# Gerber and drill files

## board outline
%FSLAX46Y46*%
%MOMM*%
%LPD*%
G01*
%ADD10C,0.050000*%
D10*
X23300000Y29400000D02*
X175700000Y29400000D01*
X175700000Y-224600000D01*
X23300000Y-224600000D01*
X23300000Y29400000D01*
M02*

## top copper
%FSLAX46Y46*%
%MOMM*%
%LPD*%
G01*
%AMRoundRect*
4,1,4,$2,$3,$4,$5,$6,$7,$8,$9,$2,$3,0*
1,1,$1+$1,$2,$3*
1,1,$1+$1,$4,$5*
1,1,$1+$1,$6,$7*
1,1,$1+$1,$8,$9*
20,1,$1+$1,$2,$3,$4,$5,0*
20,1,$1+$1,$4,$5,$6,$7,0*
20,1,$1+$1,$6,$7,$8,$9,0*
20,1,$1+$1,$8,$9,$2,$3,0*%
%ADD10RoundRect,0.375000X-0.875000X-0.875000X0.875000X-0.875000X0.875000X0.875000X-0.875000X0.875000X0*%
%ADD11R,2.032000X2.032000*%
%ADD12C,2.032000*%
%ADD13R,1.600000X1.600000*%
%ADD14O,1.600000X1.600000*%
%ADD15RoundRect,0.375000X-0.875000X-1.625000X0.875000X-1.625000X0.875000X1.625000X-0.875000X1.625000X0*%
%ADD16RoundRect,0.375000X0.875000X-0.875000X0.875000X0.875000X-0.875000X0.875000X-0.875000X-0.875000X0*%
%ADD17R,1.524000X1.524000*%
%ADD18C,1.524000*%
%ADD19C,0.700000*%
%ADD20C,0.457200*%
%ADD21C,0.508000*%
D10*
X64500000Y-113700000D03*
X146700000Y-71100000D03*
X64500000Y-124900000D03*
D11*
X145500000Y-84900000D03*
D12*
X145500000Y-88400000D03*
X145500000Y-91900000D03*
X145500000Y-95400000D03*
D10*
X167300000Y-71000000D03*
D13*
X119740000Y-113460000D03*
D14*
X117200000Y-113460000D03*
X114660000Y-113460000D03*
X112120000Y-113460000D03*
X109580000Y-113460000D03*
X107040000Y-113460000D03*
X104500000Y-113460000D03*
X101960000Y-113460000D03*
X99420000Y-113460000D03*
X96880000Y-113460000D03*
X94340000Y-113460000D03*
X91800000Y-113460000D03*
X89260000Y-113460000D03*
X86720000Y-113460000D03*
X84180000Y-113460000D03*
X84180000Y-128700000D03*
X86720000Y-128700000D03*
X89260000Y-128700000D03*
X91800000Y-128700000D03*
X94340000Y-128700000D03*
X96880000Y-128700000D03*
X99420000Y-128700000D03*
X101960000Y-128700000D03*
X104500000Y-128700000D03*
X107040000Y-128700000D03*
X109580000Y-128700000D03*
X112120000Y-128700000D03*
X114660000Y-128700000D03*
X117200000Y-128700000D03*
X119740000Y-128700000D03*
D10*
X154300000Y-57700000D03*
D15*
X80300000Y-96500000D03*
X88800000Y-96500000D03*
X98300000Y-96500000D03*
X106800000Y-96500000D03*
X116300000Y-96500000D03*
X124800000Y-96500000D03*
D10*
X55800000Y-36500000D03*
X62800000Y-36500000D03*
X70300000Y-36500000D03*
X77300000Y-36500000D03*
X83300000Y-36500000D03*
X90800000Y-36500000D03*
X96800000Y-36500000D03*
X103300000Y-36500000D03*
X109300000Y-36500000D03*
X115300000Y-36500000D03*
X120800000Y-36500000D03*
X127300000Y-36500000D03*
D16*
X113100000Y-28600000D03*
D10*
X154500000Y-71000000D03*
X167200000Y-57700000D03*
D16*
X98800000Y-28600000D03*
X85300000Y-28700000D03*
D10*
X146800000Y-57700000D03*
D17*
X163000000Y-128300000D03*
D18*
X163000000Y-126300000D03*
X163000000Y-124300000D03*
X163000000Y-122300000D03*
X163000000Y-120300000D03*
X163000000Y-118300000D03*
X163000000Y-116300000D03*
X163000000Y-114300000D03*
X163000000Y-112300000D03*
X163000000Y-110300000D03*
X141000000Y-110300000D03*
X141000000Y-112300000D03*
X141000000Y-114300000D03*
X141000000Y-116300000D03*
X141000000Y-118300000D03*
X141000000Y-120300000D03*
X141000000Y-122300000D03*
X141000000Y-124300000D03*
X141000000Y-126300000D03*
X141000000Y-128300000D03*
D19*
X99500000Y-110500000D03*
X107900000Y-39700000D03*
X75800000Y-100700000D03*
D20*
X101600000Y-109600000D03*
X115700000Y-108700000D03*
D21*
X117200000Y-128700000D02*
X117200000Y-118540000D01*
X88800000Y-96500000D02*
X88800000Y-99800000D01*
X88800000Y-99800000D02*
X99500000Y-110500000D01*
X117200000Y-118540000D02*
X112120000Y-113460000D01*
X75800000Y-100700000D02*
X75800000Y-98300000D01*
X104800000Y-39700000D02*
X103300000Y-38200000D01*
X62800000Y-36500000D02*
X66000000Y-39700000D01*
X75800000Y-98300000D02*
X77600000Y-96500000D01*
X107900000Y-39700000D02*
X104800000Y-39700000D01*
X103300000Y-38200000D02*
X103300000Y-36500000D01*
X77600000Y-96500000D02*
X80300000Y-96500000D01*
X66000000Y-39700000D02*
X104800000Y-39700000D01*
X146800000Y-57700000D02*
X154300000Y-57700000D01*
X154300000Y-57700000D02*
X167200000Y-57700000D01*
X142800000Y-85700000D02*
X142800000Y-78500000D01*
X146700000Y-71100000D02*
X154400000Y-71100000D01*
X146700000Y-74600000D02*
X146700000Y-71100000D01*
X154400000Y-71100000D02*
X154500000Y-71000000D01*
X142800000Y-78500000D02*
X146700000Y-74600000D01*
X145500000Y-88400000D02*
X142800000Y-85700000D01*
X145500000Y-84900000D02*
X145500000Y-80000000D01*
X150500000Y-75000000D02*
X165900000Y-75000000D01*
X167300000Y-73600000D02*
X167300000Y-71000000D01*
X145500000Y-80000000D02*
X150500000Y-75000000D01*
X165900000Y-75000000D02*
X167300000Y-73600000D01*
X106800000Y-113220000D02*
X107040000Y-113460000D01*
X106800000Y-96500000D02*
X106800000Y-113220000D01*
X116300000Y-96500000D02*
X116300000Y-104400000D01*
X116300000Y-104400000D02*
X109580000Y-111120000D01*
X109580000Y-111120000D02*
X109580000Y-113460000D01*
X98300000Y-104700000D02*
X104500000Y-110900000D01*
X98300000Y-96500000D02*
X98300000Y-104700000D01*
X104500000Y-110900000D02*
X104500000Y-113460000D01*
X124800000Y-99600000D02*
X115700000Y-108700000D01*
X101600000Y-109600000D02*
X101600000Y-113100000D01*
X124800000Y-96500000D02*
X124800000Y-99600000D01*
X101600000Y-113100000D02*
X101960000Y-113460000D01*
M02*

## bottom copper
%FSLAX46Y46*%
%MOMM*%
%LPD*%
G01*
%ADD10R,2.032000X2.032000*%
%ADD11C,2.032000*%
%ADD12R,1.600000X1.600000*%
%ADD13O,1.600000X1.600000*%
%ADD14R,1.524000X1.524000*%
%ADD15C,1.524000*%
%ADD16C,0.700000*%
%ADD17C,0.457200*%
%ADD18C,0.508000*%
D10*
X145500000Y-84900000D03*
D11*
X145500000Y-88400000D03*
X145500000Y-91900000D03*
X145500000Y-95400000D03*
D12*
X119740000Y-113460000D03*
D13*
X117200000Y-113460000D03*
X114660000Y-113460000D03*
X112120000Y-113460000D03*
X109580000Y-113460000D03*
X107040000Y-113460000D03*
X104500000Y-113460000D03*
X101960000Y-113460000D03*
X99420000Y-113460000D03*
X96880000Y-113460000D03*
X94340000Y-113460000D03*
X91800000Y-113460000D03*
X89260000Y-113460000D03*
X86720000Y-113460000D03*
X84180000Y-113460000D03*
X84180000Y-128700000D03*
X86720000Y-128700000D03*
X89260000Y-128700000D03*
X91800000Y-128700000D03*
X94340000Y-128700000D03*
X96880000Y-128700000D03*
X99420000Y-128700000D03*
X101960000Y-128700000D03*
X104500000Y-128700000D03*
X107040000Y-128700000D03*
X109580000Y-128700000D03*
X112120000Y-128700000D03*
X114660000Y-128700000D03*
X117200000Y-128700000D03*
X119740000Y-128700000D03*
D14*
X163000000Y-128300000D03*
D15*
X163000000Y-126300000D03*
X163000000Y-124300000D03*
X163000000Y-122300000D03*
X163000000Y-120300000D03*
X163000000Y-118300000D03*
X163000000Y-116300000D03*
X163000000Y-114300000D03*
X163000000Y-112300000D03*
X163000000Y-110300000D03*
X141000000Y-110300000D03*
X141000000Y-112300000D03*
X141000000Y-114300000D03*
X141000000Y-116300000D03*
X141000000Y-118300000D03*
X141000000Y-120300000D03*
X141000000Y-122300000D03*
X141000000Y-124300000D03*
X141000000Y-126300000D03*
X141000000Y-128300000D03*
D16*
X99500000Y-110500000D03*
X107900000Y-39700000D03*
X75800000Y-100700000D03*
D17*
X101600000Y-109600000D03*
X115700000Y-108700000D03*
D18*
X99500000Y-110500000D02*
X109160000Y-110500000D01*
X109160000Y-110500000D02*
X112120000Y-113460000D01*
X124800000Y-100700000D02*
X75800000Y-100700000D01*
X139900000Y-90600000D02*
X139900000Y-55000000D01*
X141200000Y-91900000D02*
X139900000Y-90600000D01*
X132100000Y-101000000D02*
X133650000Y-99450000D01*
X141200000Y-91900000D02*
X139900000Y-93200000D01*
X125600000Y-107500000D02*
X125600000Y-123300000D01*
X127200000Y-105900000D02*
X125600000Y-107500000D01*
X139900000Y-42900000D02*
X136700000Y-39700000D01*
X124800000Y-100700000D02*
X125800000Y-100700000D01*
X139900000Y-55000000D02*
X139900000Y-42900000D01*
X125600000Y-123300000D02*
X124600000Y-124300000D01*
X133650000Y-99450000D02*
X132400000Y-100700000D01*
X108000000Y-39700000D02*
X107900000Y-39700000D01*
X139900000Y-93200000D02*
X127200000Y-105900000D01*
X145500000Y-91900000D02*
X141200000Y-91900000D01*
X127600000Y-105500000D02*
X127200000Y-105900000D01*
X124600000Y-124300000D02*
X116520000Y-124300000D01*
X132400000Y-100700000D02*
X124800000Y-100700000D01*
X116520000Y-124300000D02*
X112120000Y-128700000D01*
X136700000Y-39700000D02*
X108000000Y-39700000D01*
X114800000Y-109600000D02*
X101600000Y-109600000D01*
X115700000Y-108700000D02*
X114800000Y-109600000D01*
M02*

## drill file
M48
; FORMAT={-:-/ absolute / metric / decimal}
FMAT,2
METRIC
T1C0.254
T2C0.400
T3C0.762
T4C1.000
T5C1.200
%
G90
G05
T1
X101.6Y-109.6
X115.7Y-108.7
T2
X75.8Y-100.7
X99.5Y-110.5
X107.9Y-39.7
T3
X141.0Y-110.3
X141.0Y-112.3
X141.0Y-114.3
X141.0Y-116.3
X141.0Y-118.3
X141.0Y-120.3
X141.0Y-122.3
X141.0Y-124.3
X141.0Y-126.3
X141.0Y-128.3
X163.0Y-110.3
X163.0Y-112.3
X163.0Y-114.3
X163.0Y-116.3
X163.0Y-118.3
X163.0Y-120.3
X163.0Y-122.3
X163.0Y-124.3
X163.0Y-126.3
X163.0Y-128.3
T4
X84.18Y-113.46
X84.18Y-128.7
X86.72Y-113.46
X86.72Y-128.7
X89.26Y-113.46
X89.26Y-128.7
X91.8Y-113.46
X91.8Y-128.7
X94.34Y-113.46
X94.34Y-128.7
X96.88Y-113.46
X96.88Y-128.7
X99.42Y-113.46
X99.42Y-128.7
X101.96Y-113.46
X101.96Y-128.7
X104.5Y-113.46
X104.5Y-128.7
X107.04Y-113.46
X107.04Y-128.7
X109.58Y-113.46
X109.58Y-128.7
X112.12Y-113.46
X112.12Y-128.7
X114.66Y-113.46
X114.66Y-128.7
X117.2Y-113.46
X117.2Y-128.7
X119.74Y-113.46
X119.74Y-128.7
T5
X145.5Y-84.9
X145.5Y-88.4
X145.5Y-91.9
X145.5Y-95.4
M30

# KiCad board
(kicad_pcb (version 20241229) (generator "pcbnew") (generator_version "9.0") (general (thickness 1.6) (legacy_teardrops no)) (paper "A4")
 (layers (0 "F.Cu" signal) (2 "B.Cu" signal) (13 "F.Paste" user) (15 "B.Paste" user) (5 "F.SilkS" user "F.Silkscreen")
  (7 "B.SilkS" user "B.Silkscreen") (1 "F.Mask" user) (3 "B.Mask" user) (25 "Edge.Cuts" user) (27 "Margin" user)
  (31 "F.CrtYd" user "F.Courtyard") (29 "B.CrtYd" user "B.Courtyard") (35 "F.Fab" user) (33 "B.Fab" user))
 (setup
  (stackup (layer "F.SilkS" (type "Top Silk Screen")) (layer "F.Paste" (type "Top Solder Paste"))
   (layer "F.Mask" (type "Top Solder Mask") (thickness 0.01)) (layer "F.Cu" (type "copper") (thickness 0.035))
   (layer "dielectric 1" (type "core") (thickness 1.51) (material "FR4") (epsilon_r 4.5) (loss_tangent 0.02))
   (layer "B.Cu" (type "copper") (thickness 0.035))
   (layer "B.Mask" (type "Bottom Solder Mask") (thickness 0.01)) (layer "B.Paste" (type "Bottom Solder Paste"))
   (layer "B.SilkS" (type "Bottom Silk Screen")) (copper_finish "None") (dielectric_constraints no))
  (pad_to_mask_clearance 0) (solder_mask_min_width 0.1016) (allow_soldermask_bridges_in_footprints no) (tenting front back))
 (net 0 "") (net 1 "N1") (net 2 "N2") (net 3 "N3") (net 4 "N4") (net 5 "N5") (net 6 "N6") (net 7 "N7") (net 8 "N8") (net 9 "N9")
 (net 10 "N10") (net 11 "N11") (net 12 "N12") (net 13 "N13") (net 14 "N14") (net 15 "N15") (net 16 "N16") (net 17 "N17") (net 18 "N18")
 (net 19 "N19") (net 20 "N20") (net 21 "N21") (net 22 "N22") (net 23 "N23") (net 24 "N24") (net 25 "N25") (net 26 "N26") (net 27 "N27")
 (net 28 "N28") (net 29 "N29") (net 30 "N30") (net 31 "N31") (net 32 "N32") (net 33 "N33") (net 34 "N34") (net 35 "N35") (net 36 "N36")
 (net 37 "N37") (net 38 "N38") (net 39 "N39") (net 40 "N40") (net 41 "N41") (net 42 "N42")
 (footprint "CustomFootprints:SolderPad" (layer "F.Cu") (at 64.5 113.7)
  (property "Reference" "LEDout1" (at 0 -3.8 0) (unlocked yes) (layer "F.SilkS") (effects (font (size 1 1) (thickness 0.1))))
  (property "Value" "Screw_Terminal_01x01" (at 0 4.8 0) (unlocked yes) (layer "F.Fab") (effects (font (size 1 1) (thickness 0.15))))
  (pad "1" smd roundrect (at 0 0) (size 2.5 2.5) (layers "F.Cu" "F.Mask" "F.Paste") (roundrect_rratio 0.15) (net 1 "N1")))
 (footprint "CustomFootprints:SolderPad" (layer "F.Cu") (at 146.7 71.1)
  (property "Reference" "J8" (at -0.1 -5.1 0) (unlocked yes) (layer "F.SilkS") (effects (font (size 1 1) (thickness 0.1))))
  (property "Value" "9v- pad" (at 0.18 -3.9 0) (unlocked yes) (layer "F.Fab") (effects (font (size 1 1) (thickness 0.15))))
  (pad "1" smd roundrect (at 0 0) (size 2.5 2.5) (layers "F.Cu" "F.Mask" "F.Paste") (roundrect_rratio 0.15) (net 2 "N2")))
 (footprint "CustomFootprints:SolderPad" (layer "F.Cu") (at 64.5 124.9)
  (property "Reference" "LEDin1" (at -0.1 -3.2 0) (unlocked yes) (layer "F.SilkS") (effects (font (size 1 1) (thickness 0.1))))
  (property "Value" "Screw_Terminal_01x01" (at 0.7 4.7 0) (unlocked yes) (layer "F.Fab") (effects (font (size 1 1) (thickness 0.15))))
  (pad "1" smd roundrect (at 0 0) (size 2.5 2.5) (layers "F.Cu" "F.Mask" "F.Paste") (roundrect_rratio 0.15) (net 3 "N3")))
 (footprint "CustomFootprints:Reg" (layer "F.Cu") (at 143.5884 104.0514)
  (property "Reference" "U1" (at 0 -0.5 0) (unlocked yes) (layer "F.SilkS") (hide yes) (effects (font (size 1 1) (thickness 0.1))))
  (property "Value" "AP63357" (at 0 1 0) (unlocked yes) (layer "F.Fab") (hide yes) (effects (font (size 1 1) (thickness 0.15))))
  (pad "1" thru_hole rect (at 1.9116 -19.1514 270) (size 2.032 2.032) (drill 1.2) (layers "*.Cu" "*.Mask") (remove_unused_layers no)
   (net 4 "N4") (solder_mask_margin 0.0635) (thermal_bridge_angle 0))
  (pad "2" thru_hole circle (at 1.9116 -15.6514 270) (size 2.032 2.032) (drill 1.2) (layers "*.Cu" "*.Mask") (remove_unused_layers no)
   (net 2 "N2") (solder_mask_margin 0.0635) (thermal_bridge_angle 0))
  (pad "3" thru_hole circle (at 1.9116 -12.1514 270) (size 2.032 2.032) (drill 1.2) (layers "*.Cu" "*.Mask") (remove_unused_layers no)
   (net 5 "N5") (solder_mask_margin 0.0635) (thermal_bridge_angle 0))
  (pad "4" thru_hole circle (at 1.9116 -8.6514 270) (size 2.032 2.032) (drill 1.2) (layers "*.Cu" "*.Mask") (remove_unused_layers no)
   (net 1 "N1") (solder_mask_margin 0.0635) (thermal_bridge_angle 0)))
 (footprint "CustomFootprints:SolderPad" (layer "F.Cu") (at 167.3 71)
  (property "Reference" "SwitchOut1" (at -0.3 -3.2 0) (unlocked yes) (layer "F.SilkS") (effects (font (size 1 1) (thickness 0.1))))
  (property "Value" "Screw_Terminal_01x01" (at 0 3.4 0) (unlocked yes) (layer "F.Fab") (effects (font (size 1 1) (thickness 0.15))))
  (pad "1" smd roundrect (at 0 0) (size 2.5 2.5) (layers "F.Cu" "F.Mask" "F.Paste") (roundrect_rratio 0.15) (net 4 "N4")))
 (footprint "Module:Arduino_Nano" (layer "F.Cu") (at 119.74 113.46 -90)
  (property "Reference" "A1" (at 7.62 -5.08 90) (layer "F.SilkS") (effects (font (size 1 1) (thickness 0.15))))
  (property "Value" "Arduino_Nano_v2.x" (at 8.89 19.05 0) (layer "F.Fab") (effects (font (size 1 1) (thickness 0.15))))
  (pad "1" thru_hole rect (at 0 0 270) (size 1.6 1.6) (drill 1) (layers "*.Cu" "*.Mask") (remove_unused_layers no) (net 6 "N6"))
  (pad "2" thru_hole oval (at 0 2.54 270) (size 1.6 1.6) (drill 1) (layers "*.Cu" "*.Mask") (remove_unused_layers no) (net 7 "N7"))
  (pad "3" thru_hole oval (at 0 5.08 270) (size 1.6 1.6) (drill 1) (layers "*.Cu" "*.Mask") (remove_unused_layers no) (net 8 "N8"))
  (pad "4" thru_hole oval (at 0 7.62 270) (size 1.6 1.6) (drill 1) (layers "*.Cu" "*.Mask") (remove_unused_layers no) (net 1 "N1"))
  (pad "5" thru_hole oval (at 0 10.16 270) (size 1.6 1.6) (drill 1) (layers "*.Cu" "*.Mask") (remove_unused_layers no) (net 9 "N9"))
  (pad "6" thru_hole oval (at 0 12.7 270) (size 1.6 1.6) (drill 1) (layers "*.Cu" "*.Mask") (remove_unused_layers no) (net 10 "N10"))
  (pad "7" thru_hole oval (at 0 15.24 270) (size 1.6 1.6) (drill 1) (layers "*.Cu" "*.Mask") (remove_unused_layers no) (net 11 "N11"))
  (pad "8" thru_hole oval (at 0 17.78 270) (size 1.6 1.6) (drill 1) (layers "*.Cu" "*.Mask") (remove_unused_layers no) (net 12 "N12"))
  (pad "9" thru_hole oval (at 0 20.32 270) (size 1.6 1.6) (drill 1) (layers "*.Cu" "*.Mask") (remove_unused_layers no) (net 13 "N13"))
  (pad "10" thru_hole oval (at 0 22.86 270) (size 1.6 1.6) (drill 1) (layers "*.Cu" "*.Mask") (remove_unused_layers no) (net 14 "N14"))
  (pad "11" thru_hole oval (at 0 25.4 270) (size 1.6 1.6) (drill 1) (layers "*.Cu" "*.Mask") (remove_unused_layers no) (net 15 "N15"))
  (pad "12" thru_hole oval (at 0 27.94 270) (size 1.6 1.6) (drill 1) (layers "*.Cu" "*.Mask") (remove_unused_layers no) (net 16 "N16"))
  (pad "13" thru_hole oval (at 0 30.48 270) (size 1.6 1.6) (drill 1) (layers "*.Cu" "*.Mask") (remove_unused_layers no) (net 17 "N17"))
  (pad "14" thru_hole oval (at 0 33.02 270) (size 1.6 1.6) (drill 1) (layers "*.Cu" "*.Mask") (remove_unused_layers no) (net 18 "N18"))
  (pad "15" thru_hole oval (at 0 35.56 270) (size 1.6 1.6) (drill 1) (layers "*.Cu" "*.Mask") (remove_unused_layers no) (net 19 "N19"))
  (pad "16" thru_hole oval (at 15.24 35.56 270) (size 1.6 1.6) (drill 1) (layers "*.Cu" "*.Mask") (remove_unused_layers no) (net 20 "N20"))
  (pad "17" thru_hole oval (at 15.24 33.02 270) (size 1.6 1.6) (drill 1) (layers "*.Cu" "*.Mask") (remove_unused_layers no) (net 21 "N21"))
  (pad "18" thru_hole oval (at 15.24 30.48 270) (size 1.6 1.6) (drill 1) (layers "*.Cu" "*.Mask") (remove_unused_layers no) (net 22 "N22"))
  (pad "19" thru_hole oval (at 15.24 27.94 270) (size 1.6 1.6) (drill 1) (layers "*.Cu" "*.Mask") (remove_unused_layers no) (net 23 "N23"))
  (pad "20" thru_hole oval (at 15.24 25.4 270) (size 1.6 1.6) (drill 1) (layers "*.Cu" "*.Mask") (remove_unused_layers no) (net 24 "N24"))
  (pad "21" thru_hole oval (at 15.24 22.86 270) (size 1.6 1.6) (drill 1) (layers "*.Cu" "*.Mask") (remove_unused_layers no) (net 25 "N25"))
  (pad "22" thru_hole oval (at 15.24 20.32 270) (size 1.6 1.6) (drill 1) (layers "*.Cu" "*.Mask") (remove_unused_layers no) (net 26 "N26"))
  (pad "23" thru_hole oval (at 15.24 17.78 270) (size 1.6 1.6) (drill 1) (layers "*.Cu" "*.Mask") (remove_unused_layers no) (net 3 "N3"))
  (pad "24" thru_hole oval (at 15.24 15.24 270) (size 1.6 1.6) (drill 1) (layers "*.Cu" "*.Mask") (remove_unused_layers no) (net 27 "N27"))
  (pad "25" thru_hole oval (at 15.24 12.7 270) (size 1.6 1.6) (drill 1) (layers "*.Cu" "*.Mask") (remove_unused_layers no) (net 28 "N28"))
  (pad "26" thru_hole oval (at 15.24 10.16 270) (size 1.6 1.6) (drill 1) (layers "*.Cu" "*.Mask") (remove_unused_layers no) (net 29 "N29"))
  (pad "27" thru_hole oval (at 15.24 7.62 270) (size 1.6 1.6) (drill 1) (layers "*.Cu" "*.Mask") (remove_unused_layers no) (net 5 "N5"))
  (pad "28" thru_hole oval (at 15.24 5.08 270) (size 1.6 1.6) (drill 1) (layers "*.Cu" "*.Mask") (remove_unused_layers no) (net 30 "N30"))
  (pad "29" thru_hole oval (at 15.24 2.54 270) (size 1.6 1.6) (drill 1) (layers "*.Cu" "*.Mask") (remove_unused_layers no) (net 1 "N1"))
  (pad "30" thru_hole oval (at 15.24 0 270) (size 1.6 1.6) (drill 1) (layers "*.Cu" "*.Mask") (remove_unused_layers no) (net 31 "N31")))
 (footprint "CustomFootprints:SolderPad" (layer "F.Cu") (at 154.3 57.7)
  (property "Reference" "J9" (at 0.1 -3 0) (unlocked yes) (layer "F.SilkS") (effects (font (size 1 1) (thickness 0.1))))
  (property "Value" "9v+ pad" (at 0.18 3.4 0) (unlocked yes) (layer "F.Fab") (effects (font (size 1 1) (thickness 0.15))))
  (pad "1" smd roundrect (at 0 0) (size 2.5 2.5) (layers "F.Cu" "F.Mask" "F.Paste") (roundrect_rratio 0.15) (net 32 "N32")))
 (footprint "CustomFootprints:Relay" (layer "F.Cu") (at 90.8 66)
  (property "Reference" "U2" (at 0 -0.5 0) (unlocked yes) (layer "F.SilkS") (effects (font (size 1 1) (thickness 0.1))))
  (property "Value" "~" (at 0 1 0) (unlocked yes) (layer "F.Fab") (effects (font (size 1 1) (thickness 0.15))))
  (pad "1" smd roundrect (at -10.5 30.5) (size 2.5 4) (layers "F.Cu" "F.Mask" "F.Paste") (roundrect_rratio 0.15) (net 5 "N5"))
  (pad "2" smd roundrect (at -2 30.5) (size 2.5 4) (layers "F.Cu" "F.Mask" "F.Paste") (roundrect_rratio 0.15) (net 1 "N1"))
  (pad "3" smd roundrect (at 7.5 30.5) (size 2.5 4) (layers "F.Cu" "F.Mask" "F.Paste") (roundrect_rratio 0.15) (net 11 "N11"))
  (pad "4" smd roundrect (at 16 30.5) (size 2.5 4) (layers "F.Cu" "F.Mask" "F.Paste") (roundrect_rratio 0.15) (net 10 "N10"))
  (pad "5" smd roundrect (at 25.5 30.5) (size 2.5 4) (layers "F.Cu" "F.Mask" "F.Paste") (roundrect_rratio 0.15) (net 9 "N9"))
  (pad "6" smd roundrect (at 34 30.5) (size 2.5 4) (layers "F.Cu" "F.Mask" "F.Paste") (roundrect_rratio 0.15) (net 12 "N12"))
  (pad "7" smd roundrect (at -35 -29.5) (size 2.5 2.5) (layers "F.Cu" "F.Mask" "F.Paste") (roundrect_rratio 0.15) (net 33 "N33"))
  (pad "8" smd roundrect (at -28 -29.5) (size 2.5 2.5) (layers "F.Cu" "F.Mask" "F.Paste") (roundrect_rratio 0.15) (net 5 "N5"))
  (pad "9" smd roundrect (at -20.5 -29.5) (size 2.5 2.5) (layers "F.Cu" "F.Mask" "F.Paste") (roundrect_rratio 0.15) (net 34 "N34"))
  (pad "10" smd roundrect (at -13.5 -29.5) (size 2.5 2.5) (layers "F.Cu" "F.Mask" "F.Paste") (roundrect_rratio 0.15) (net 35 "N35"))
  (pad "11" smd roundrect (at -7.5 -29.5) (size 2.5 2.5) (layers "F.Cu" "F.Mask" "F.Paste") (roundrect_rratio 0.15) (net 5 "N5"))
  (pad "12" smd roundrect (at 0 -29.5) (size 2.5 2.5) (layers "F.Cu" "F.Mask" "F.Paste") (roundrect_rratio 0.15) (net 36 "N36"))
  (pad "13" smd roundrect (at 6 -29.5) (size 2.5 2.5) (layers "F.Cu" "F.Mask" "F.Paste") (roundrect_rratio 0.15) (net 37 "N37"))
  (pad "14" smd roundrect (at 12.5 -29.5) (size 2.5 2.5) (layers "F.Cu" "F.Mask" "F.Paste") (roundrect_rratio 0.15) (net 5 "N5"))
  (pad "15" smd roundrect (at 18.5 -29.5) (size 2.5 2.5) (layers "F.Cu" "F.Mask" "F.Paste") (roundrect_rratio 0.15) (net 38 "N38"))
  (pad "16" smd roundrect (at 24.5 -29.5) (size 2.5 2.5) (layers "F.Cu" "F.Mask" "F.Paste") (roundrect_rratio 0.15) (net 36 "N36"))
  (pad "17" smd roundrect (at 30 -29.5) (size 2.5 2.5) (layers "F.Cu" "F.Mask" "F.Paste") (roundrect_rratio 0.15) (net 1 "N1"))
  (pad "18" smd roundrect (at 36.5 -29.5) (size 2.5 2.5) (layers "F.Cu" "F.Mask" "F.Paste") (roundrect_rratio 0.15) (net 38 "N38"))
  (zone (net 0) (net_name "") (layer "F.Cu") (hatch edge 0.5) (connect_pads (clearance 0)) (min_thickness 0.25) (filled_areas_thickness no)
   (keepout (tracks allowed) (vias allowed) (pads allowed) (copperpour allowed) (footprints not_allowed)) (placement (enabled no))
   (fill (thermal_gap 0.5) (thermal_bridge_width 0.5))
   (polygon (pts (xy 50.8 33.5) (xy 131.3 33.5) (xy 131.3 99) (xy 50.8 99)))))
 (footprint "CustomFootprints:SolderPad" (layer "F.Cu") (at 113.1 28.6 90)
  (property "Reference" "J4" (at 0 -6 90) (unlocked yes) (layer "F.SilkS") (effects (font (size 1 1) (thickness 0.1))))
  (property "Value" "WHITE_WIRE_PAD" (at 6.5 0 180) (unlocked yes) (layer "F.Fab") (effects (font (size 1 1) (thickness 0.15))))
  (pad "1" smd roundrect (at 0 0 90) (size 2.5 2.5) (layers "F.Cu" "F.Mask" "F.Paste") (roundrect_rratio 0.15) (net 38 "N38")))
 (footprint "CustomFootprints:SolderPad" (layer "F.Cu") (at 154.5 71)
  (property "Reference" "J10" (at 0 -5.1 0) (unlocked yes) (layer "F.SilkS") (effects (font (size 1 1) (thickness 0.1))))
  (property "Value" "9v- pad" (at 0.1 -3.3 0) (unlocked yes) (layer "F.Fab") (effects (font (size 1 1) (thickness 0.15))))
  (pad "1" smd roundrect (at 0 0) (size 2.5 2.5) (layers "F.Cu" "F.Mask" "F.Paste") (roundrect_rratio 0.15) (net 2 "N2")))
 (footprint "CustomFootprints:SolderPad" (layer "F.Cu") (at 167.2 57.7)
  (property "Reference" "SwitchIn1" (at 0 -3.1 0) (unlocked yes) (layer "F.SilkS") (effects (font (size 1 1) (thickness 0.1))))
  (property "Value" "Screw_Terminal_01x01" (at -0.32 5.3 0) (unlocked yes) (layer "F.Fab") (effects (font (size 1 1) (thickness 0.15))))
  (pad "1" smd roundrect (at 0 0) (size 2.5 2.5) (layers "F.Cu" "F.Mask" "F.Paste") (roundrect_rratio 0.15) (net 32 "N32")))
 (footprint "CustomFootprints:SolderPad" (layer "F.Cu") (at 98.8 28.6 90)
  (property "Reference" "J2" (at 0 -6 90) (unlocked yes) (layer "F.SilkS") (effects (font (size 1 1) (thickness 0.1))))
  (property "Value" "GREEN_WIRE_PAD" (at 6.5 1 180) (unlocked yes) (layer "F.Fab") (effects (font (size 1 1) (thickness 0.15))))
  (pad "1" smd roundrect (at 0 0 90) (size 2.5 2.5) (layers "F.Cu" "F.Mask" "F.Paste") (roundrect_rratio 0.15) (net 34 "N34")))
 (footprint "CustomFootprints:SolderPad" (layer "F.Cu") (at 85.3 28.7 90)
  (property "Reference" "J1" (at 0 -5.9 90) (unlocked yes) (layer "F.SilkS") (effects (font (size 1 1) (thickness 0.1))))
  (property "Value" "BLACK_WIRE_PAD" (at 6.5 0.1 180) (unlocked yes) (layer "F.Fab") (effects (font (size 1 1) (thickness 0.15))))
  (pad "1" smd roundrect (at 0 0 90) (size 2.5 2.5) (layers "F.Cu" "F.Mask" "F.Paste") (roundrect_rratio 0.15) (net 36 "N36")))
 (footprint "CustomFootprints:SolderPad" (layer "F.Cu") (at 146.8 57.7)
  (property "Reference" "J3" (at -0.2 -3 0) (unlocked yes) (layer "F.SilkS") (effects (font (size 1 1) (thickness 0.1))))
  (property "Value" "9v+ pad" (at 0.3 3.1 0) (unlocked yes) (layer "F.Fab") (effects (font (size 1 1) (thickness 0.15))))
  (pad "1" smd roundrect (at 0 0) (size 2.5 2.5) (layers "F.Cu" "F.Mask" "F.Paste") (roundrect_rratio 0.15) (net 32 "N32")))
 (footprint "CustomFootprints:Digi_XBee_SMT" (layer "F.Cu") (at 164.19 108.29 180)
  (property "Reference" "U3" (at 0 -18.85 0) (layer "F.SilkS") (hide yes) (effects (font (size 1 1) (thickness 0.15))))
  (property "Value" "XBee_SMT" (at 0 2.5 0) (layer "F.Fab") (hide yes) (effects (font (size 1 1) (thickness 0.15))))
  (pad "1" thru_hole rect (at 1.19 -20.01 180) (size 1.524 1.524) (drill 0.762) (layers "*.Cu" "*.Mask") (remove_unused_layers no)
   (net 1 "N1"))
  (pad "2" thru_hole circle (at 1.19 -18.01 180) (size 1.524 1.524) (drill 0.762) (layers "*.Cu" "*.Mask") (remove_unused_layers no)
   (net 5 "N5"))
  (pad "3" thru_hole circle (at 1.19 -16.01 180) (size 1.524 1.524) (drill 0.762) (layers "*.Cu" "*.Mask") (remove_unused_layers no)
   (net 18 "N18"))
  (pad "4" thru_hole circle (at 1.19 -14.01 180) (size 1.524 1.524) (drill 0.762) (layers "*.Cu" "*.Mask") (remove_unused_layers no)
   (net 17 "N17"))
  (pad "5" thru_hole circle (at 1.19 -12.01 180) (size 1.524 1.524) (drill 0.762) (layers "*.Cu" "*.Mask") (remove_unused_layers no))
  (pad "6" thru_hole circle (at 1.19 -10.01 180) (size 1.524 1.524) (drill 0.762) (layers "*.Cu" "*.Mask") (remove_unused_layers no))
  (pad "7" thru_hole circle (at 1.19 -8.01 180) (size 1.524 1.524) (drill 0.762) (layers "*.Cu" "*.Mask") (remove_unused_layers no))
  (pad "8" thru_hole circle (at 1.19 -6.01 180) (size 1.524 1.524) (drill 0.762) (layers "*.Cu" "*.Mask") (remove_unused_layers no))
  (pad "9" thru_hole circle (at 1.19 -4.01 180) (size 1.524 1.524) (drill 0.762) (layers "*.Cu" "*.Mask") (remove_unused_layers no)
   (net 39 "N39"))
  (pad "10" thru_hole circle (at 1.19 -2.01 180) (size 1.524 1.524) (drill 0.762) (layers "*.Cu" "*.Mask") (remove_unused_layers no))
  (pad "11" thru_hole circle (at 23.19 -2.01 180) (size 1.524 1.524) (drill 0.762) (layers "*.Cu" "*.Mask") (remove_unused_layers no))
  (pad "12" thru_hole circle (at 23.19 -4.01 180) (size 1.524 1.524) (drill 0.762) (layers "*.Cu" "*.Mask") (remove_unused_layers no))
  (pad "13" thru_hole circle (at 23.19 -6.01 180) (size 1.524 1.524) (drill 0.762) (layers "*.Cu" "*.Mask") (remove_unused_layers no))
  (pad "14" thru_hole circle (at 23.19 -8.01 180) (size 1.524 1.524) (drill 0.762) (layers "*.Cu" "*.Mask") (remove_unused_layers no))
  (pad "15" thru_hole circle (at 23.19 -10.01 180) (size 1.524 1.524) (drill 0.762) (layers "*.Cu" "*.Mask") (remove_unused_layers no))
  (pad "16" thru_hole circle (at 23.19 -12.01 180) (size 1.524 1.524) (drill 0.762) (layers "*.Cu" "*.Mask") (remove_unused_layers no))
  (pad "17" thru_hole circle (at 23.19 -14.01 180) (size 1.524 1.524) (drill 0.762) (layers "*.Cu" "*.Mask") (remove_unused_layers no))
  (pad "18" thru_hole circle (at 23.19 -16.01 180) (size 1.524 1.524) (drill 0.762) (layers "*.Cu" "*.Mask") (remove_unused_layers no)
   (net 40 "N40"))
  (pad "19" thru_hole circle (at 23.19 -18.01 180) (size 1.524 1.524) (drill 0.762) (layers "*.Cu" "*.Mask") (remove_unused_layers no)
   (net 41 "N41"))
  (pad "20" thru_hole circle (at 23.19 -20.01 180) (size 1.524 1.524) (drill 0.762) (layers "*.Cu" "*.Mask") (remove_unused_layers no)
   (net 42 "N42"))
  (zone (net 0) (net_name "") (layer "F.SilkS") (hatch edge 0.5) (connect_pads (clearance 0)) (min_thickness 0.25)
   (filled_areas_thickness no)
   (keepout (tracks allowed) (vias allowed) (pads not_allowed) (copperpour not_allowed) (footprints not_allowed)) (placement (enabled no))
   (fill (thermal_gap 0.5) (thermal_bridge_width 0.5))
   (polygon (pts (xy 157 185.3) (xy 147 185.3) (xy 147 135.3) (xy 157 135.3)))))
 (gr_rect (start 23.3 -29.4) (end 175.7 224.6) (stroke (width 0.05) (type solid)) (fill no) (layer "Edge.Cuts"))
 (segment (start 117.2 128.7) (end 117.2 118.54) (width 0.508) (layer "F.Cu") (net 1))
 (segment (start 88.8 96.5) (end 88.8 99.8) (width 0.508) (layer "F.Cu") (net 1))
 (segment (start 88.8 99.8) (end 99.5 110.5) (width 0.508) (layer "F.Cu") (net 1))
 (segment (start 117.2 118.54) (end 112.12 113.46) (width 0.508) (layer "F.Cu") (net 1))
 (via (at 99.5 110.5) (size 0.7) (drill 0.4) (layers "F.Cu" "B.Cu") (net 1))
 (segment (start 99.5 110.5) (end 109.16 110.5) (width 0.508) (layer "B.Cu") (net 1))
 (segment (start 109.16 110.5) (end 112.12 113.46) (width 0.508) (layer "B.Cu") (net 1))
 (segment (start 75.8 100.7) (end 75.8 98.3) (width 0.508) (layer "F.Cu") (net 5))
 (segment (start 104.8 39.7) (end 103.3 38.2) (width 0.508) (layer "F.Cu") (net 5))
 (segment (start 62.8 36.5) (end 66 39.7) (width 0.508) (layer "F.Cu") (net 5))
 (segment (start 75.8 98.3) (end 77.6 96.5) (width 0.508) (layer "F.Cu") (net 5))
 (segment (start 107.9 39.7) (end 104.8 39.7) (width 0.508) (layer "F.Cu") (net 5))
 (segment (start 103.3 38.2) (end 103.3 36.5) (width 0.508) (layer "F.Cu") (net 5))
 (segment (start 77.6 96.5) (end 80.3 96.5) (width 0.508) (layer "F.Cu") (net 5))
 (segment (start 66 39.7) (end 104.8 39.7) (width 0.508) (layer "F.Cu") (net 5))
 (via (at 107.9 39.7) (size 0.7) (drill 0.4) (layers "F.Cu" "B.Cu") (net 5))
 (via (at 75.8 100.7) (size 0.7) (drill 0.4) (layers "F.Cu" "B.Cu") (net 5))
 (segment (start 124.8 100.7) (end 75.8 100.7) (width 0.508) (layer "B.Cu") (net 5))
 (segment (start 139.9 90.6) (end 139.9 55) (width 0.508) (layer "B.Cu") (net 5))
 (segment (start 141.2 91.9) (end 139.9 90.6) (width 0.508) (layer "B.Cu") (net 5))
 (segment (start 132.1 101) (end 133.65 99.45) (width 0.508) (layer "B.Cu") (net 5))
 (segment (start 141.2 91.9) (end 139.9 93.2) (width 0.508) (layer "B.Cu") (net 5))
 (segment (start 125.6 107.5) (end 125.6 123.3) (width 0.508) (layer "B.Cu") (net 5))
 (segment (start 127.2 105.9) (end 125.6 107.5) (width 0.508) (layer "B.Cu") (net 5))
 (segment (start 139.9 42.9) (end 136.7 39.7) (width 0.508) (layer "B.Cu") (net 5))
 (segment (start 124.8 100.7) (end 125.8 100.7) (width 0.508) (layer "B.Cu") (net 5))
 (segment (start 139.9 55) (end 139.9 42.9) (width 0.508) (layer "B.Cu") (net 5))
 (segment (start 125.6 123.3) (end 124.6 124.3) (width 0.508) (layer "B.Cu") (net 5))
 (segment (start 133.65 99.45) (end 132.4 100.7) (width 0.508) (layer "B.Cu") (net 5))
 (segment (start 108 39.7) (end 107.9 39.7) (width 0.508) (layer "B.Cu") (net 5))
 (segment (start 139.9 93.2) (end 127.2 105.9) (width 0.508) (layer "B.Cu") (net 5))
 (segment (start 145.5 91.9) (end 141.2 91.9) (width 0.508) (layer "B.Cu") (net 5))
 (segment (start 127.6 105.5) (end 127.2 105.9) (width 0.508) (layer "B.Cu") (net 5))
 (segment (start 124.6 124.3) (end 116.52 124.3) (width 0.508) (layer "B.Cu") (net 5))
 (segment (start 132.4 100.7) (end 124.8 100.7) (width 0.508) (layer "B.Cu") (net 5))
 (segment (start 116.52 124.3) (end 112.12 128.7) (width 0.508) (layer "B.Cu") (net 5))
 (segment (start 136.7 39.7) (end 108 39.7) (width 0.508) (layer "B.Cu") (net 5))
 (segment (start 146.8 57.7) (end 154.3 57.7) (width 0.508) (layer "F.Cu") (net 32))
 (segment (start 154.3 57.7) (end 167.2 57.7) (width 0.508) (layer "F.Cu") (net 32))
 (segment (start 142.8 85.7) (end 142.8 78.5) (width 0.508) (layer "F.Cu") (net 2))
 (segment (start 146.7 71.1) (end 154.4 71.1) (width 0.508) (layer "F.Cu") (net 2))
 (segment (start 146.7 74.6) (end 146.7 71.1) (width 0.508) (layer "F.Cu") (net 2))
 (segment (start 154.4 71.1) (end 154.5 71) (width 0.508) (layer "F.Cu") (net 2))
 (segment (start 142.8 78.5) (end 146.7 74.6) (width 0.508) (layer "F.Cu") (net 2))
 (segment (start 145.5 88.4) (end 142.8 85.7) (width 0.508) (layer "F.Cu") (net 2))
 (segment (start 145.5 84.9) (end 145.5 80) (width 0.508) (layer "F.Cu") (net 4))
 (segment (start 150.5 75) (end 165.9 75) (width 0.508) (layer "F.Cu") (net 4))
 (segment (start 167.3 73.6) (end 167.3 71) (width 0.508) (layer "F.Cu") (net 4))
 (segment (start 145.5 80) (end 150.5 75) (width 0.508) (layer "F.Cu") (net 4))
 (segment (start 165.9 75) (end 167.3 73.6) (width 0.508) (layer "F.Cu") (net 4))
 (segment (start 106.8 113.22) (end 107.04 113.46) (width 0.508) (layer "F.Cu") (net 10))
 (segment (start 106.8 96.5) (end 106.8 113.22) (width 0.508) (layer "F.Cu") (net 10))
 (segment (start 116.3 96.5) (end 116.3 104.4) (width 0.508) (layer "F.Cu") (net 9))
 (segment (start 116.3 104.4) (end 109.58 111.12) (width 0.508) (layer "F.Cu") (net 9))
 (segment (start 109.58 111.12) (end 109.58 113.46) (width 0.508) (layer "F.Cu") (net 9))
 (segment (start 98.3 104.7) (end 104.5 110.9) (width 0.508) (layer "F.Cu") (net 11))
 (segment (start 98.3 96.5) (end 98.3 104.7) (width 0.508) (layer "F.Cu") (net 11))
 (segment (start 104.5 110.9) (end 104.5 113.46) (width 0.508) (layer "F.Cu") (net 11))
 (segment (start 124.8 99.6) (end 115.7 108.7) (width 0.508) (layer "F.Cu") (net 12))
 (segment (start 101.6 109.6) (end 101.6 113.1) (width 0.508) (layer "F.Cu") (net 12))
 (segment (start 124.8 96.5) (end 124.8 99.6) (width 0.508) (layer "F.Cu") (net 12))
 (segment (start 101.6 113.1) (end 101.96 113.46) (width 0.508) (layer "F.Cu") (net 12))
 (via (at 101.6 109.6) (size 0.4572) (drill 0.254) (layers "F.Cu" "B.Cu") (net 12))
 (via (at 115.7 108.7) (size 0.4572) (drill 0.254) (layers "F.Cu" "B.Cu") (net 12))
 (segment (start 114.8 109.6) (end 101.6 109.6) (width 0.508) (layer "B.Cu") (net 12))
 (segment (start 115.7 108.7) (end 114.8 109.6) (width 0.508) (layer "B.Cu") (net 12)))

